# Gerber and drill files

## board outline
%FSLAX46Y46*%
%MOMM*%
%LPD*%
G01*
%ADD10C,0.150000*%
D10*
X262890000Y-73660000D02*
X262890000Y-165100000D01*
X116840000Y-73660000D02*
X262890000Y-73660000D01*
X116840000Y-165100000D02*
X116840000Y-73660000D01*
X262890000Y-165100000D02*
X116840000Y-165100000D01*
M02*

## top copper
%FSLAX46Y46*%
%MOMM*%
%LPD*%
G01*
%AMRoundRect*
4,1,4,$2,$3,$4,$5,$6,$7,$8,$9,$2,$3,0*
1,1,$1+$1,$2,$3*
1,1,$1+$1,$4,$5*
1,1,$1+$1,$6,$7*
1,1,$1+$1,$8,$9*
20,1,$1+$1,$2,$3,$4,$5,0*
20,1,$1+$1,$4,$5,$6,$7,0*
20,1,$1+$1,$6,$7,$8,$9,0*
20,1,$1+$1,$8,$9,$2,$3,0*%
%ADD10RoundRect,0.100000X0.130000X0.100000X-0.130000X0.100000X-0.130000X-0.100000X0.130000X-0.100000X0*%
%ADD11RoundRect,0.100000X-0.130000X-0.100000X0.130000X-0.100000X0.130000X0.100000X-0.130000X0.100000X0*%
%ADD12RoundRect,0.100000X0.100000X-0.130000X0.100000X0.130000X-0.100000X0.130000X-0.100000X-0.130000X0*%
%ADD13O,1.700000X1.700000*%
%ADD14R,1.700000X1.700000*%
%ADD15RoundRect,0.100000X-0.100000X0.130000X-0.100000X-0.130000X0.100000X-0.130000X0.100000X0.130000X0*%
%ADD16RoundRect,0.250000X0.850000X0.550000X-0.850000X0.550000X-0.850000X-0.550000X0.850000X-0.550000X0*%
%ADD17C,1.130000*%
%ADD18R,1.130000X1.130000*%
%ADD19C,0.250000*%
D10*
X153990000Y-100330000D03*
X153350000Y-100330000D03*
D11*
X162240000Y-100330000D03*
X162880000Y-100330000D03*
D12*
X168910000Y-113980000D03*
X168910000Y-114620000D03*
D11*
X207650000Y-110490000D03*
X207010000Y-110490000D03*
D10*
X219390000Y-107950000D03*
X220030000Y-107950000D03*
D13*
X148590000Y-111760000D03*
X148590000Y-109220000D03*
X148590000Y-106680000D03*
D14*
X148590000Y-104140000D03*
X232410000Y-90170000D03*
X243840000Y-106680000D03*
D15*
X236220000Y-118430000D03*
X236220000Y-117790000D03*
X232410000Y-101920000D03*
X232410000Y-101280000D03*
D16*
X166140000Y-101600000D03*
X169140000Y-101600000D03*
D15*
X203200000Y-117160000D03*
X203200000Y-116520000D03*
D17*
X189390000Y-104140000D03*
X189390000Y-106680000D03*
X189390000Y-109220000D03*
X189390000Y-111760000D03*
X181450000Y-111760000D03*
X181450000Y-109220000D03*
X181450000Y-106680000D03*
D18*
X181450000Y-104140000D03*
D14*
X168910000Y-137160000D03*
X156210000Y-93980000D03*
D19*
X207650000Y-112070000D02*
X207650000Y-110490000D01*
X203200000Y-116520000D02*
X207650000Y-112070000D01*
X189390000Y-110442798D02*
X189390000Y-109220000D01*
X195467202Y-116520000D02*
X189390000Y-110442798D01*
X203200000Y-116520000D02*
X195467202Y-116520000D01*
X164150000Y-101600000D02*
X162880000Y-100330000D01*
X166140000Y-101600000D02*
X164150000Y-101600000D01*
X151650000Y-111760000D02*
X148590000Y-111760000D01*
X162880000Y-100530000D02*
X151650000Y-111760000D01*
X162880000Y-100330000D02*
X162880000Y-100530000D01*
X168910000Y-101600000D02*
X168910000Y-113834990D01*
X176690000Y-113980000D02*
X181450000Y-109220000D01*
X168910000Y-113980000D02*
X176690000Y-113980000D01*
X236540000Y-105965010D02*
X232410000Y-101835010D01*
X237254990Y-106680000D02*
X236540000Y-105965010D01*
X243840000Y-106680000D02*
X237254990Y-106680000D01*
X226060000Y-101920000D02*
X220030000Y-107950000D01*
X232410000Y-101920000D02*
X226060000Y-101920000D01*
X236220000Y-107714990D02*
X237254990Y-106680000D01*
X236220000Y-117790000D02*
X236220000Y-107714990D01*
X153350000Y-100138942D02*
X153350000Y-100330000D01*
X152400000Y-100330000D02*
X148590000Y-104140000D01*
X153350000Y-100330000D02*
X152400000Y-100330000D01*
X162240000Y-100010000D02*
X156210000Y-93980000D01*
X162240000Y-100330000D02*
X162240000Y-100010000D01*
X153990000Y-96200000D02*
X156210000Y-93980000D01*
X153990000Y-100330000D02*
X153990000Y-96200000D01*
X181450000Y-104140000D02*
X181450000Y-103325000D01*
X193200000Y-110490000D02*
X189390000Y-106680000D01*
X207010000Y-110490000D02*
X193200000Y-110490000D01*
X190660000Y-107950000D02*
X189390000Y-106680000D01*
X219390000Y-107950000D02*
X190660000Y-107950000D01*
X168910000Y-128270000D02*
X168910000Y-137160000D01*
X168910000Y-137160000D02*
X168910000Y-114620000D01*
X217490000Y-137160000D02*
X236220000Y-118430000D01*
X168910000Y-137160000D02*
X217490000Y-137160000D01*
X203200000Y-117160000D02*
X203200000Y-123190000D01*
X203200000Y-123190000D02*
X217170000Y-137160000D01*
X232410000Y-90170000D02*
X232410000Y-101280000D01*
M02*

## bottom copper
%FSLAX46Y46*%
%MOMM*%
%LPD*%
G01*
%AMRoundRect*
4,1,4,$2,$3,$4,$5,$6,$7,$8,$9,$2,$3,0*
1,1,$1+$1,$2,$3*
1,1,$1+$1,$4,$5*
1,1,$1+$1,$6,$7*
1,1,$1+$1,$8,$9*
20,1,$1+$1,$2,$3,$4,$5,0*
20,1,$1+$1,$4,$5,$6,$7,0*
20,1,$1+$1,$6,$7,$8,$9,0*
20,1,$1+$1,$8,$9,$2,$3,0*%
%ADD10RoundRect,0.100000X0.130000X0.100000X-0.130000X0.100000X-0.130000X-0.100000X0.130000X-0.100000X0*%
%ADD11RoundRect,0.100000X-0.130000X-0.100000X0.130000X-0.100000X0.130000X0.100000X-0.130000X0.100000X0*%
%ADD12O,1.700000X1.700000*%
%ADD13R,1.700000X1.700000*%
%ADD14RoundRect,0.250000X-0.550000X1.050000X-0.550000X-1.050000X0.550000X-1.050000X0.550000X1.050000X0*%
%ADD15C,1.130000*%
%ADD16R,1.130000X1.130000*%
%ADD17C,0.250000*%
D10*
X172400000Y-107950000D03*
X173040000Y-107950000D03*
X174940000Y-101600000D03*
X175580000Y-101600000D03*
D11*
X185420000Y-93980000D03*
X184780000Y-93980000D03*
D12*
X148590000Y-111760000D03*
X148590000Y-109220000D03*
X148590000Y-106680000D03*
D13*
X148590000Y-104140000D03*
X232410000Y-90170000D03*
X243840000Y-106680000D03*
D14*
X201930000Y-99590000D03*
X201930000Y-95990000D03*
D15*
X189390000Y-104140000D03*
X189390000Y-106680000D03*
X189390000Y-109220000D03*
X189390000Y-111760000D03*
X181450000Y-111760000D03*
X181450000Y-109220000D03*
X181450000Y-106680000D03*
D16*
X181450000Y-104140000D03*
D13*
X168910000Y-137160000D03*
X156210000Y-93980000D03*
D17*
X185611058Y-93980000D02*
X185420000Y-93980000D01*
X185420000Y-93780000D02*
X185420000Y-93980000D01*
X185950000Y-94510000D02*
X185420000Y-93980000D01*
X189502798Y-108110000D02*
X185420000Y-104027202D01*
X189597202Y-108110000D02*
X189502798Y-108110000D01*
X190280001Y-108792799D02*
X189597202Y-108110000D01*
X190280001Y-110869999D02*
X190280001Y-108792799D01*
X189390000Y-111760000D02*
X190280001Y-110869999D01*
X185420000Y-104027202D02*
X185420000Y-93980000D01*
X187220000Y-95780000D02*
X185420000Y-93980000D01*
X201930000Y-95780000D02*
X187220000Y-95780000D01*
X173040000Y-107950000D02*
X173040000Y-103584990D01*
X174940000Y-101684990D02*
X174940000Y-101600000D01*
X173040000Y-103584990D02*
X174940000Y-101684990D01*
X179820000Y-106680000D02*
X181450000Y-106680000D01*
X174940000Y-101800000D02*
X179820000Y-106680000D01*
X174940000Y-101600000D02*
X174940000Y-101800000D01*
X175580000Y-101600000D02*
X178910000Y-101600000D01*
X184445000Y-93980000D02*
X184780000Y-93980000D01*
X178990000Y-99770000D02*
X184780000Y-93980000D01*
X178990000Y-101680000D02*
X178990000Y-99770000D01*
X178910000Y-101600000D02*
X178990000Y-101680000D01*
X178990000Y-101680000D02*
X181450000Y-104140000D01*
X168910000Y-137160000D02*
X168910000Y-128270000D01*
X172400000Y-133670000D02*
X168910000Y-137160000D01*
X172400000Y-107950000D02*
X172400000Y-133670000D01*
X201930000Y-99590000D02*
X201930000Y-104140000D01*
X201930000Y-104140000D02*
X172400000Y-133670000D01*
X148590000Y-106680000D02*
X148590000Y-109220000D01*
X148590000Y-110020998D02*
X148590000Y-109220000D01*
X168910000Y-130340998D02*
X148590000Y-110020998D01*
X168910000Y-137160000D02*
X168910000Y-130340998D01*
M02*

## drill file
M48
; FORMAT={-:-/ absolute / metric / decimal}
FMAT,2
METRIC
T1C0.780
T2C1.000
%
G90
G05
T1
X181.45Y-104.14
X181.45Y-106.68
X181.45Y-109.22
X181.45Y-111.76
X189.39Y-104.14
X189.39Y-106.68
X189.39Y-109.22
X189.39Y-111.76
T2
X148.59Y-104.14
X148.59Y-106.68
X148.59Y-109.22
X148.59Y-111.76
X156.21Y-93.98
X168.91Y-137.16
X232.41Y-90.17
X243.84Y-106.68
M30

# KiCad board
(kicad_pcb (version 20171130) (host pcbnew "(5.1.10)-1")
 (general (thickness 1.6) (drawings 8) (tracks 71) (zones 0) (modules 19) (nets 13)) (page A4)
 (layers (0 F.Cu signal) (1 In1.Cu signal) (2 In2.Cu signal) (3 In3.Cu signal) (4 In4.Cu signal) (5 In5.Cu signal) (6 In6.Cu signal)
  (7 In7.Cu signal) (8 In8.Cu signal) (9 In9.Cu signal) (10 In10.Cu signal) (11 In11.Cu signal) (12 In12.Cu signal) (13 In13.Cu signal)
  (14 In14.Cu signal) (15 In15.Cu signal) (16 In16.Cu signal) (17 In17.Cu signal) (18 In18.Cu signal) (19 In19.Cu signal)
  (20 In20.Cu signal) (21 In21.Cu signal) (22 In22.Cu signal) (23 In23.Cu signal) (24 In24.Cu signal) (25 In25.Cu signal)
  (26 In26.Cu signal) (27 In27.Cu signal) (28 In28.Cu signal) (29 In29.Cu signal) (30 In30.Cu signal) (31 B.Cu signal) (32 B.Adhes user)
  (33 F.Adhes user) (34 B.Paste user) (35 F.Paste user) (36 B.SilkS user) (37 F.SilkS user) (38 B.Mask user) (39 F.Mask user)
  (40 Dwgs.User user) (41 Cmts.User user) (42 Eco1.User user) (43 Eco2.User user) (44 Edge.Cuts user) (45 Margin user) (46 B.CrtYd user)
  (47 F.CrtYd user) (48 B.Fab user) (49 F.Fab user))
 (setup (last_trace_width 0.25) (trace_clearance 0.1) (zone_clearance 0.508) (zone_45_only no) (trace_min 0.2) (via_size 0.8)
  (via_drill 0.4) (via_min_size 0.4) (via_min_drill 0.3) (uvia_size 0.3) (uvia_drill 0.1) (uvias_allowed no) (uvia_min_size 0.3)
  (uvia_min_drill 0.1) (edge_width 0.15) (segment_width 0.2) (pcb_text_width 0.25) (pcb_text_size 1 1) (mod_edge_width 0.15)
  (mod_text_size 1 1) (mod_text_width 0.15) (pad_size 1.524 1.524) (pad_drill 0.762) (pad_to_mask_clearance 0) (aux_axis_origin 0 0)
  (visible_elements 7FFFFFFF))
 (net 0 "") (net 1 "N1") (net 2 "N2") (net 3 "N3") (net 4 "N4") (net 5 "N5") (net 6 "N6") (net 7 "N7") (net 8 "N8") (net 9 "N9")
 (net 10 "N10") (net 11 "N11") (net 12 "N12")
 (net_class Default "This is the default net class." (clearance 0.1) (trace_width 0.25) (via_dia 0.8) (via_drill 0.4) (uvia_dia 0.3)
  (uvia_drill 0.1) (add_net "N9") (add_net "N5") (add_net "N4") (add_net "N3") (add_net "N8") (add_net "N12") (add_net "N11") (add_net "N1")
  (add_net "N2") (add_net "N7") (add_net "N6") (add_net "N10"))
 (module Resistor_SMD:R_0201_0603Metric (layer F.Cu) (at 153.67 100.33 180)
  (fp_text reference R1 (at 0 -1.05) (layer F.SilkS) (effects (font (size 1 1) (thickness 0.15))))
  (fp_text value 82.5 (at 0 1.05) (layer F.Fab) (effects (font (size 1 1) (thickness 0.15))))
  (pad "" smd roundrect (at -0.345 0 180) (size 0.318 0.36) (layers F.Paste) (roundrect_rratio 0.25))
  (pad "" smd roundrect (at 0.345 0 180) (size 0.318 0.36) (layers F.Paste) (roundrect_rratio 0.25))
  (pad 1 smd roundrect (at -0.32 0 180) (size 0.46 0.4) (layers F.Cu F.Mask) (roundrect_rratio 0.25) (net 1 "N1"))
  (pad 2 smd roundrect (at 0.32 0 180) (size 0.46 0.4) (layers F.Cu F.Mask) (roundrect_rratio 0.25) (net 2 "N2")))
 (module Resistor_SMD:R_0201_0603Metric (layer F.Cu) (at 162.56 100.33)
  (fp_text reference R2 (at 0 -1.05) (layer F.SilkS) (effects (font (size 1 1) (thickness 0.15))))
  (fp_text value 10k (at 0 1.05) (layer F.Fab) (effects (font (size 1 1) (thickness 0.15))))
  (pad "" smd roundrect (at -0.345 0) (size 0.318 0.36) (layers F.Paste) (roundrect_rratio 0.25))
  (pad "" smd roundrect (at 0.345 0) (size 0.318 0.36) (layers F.Paste) (roundrect_rratio 0.25))
  (pad 1 smd roundrect (at -0.32 0) (size 0.46 0.4) (layers F.Cu F.Mask) (roundrect_rratio 0.25) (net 1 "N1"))
  (pad 2 smd roundrect (at 0.32 0) (size 0.46 0.4) (layers F.Cu F.Mask) (roundrect_rratio 0.25) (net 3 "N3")))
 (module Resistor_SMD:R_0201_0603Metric (layer F.Cu) (at 168.91 114.3 90)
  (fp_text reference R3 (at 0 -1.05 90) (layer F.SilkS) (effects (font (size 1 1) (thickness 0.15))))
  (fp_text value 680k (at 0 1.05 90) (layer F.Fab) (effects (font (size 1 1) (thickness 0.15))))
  (pad 2 smd roundrect (at 0.32 0 90) (size 0.46 0.4) (layers F.Cu F.Mask) (roundrect_rratio 0.25) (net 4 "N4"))
  (pad 1 smd roundrect (at -0.32 0 90) (size 0.46 0.4) (layers F.Cu F.Mask) (roundrect_rratio 0.25) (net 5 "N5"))
  (pad "" smd roundrect (at 0.345 0 90) (size 0.318 0.36) (layers F.Paste) (roundrect_rratio 0.25))
  (pad "" smd roundrect (at -0.345 0 90) (size 0.318 0.36) (layers F.Paste) (roundrect_rratio 0.25)))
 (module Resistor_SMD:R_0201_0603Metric (layer B.Cu) (at 172.72 107.95 180)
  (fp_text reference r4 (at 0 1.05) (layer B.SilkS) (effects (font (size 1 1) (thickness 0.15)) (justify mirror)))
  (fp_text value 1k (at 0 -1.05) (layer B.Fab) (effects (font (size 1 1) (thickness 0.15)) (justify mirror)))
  (pad 2 smd roundrect (at 0.32 0 180) (size 0.46 0.4) (layers B.Cu B.Mask) (roundrect_rratio 0.25) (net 5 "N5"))
  (pad 1 smd roundrect (at -0.32 0 180) (size 0.46 0.4) (layers B.Cu B.Mask) (roundrect_rratio 0.25) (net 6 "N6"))
  (pad "" smd roundrect (at 0.345 0 180) (size 0.318 0.36) (layers B.Paste) (roundrect_rratio 0.25))
  (pad "" smd roundrect (at -0.345 0 180) (size 0.318 0.36) (layers B.Paste) (roundrect_rratio 0.25)))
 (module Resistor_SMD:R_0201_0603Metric (layer B.Cu) (at 175.26 101.6 180)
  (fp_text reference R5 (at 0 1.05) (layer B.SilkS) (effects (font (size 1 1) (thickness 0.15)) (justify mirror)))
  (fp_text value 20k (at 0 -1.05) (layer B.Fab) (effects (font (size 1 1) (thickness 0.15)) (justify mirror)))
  (pad 2 smd roundrect (at 0.32 0 180) (size 0.46 0.4) (layers B.Cu B.Mask) (roundrect_rratio 0.25) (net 6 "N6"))
  (pad 1 smd roundrect (at -0.32 0 180) (size 0.46 0.4) (layers B.Cu B.Mask) (roundrect_rratio 0.25) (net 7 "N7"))
  (pad "" smd roundrect (at 0.345 0 180) (size 0.318 0.36) (layers B.Paste) (roundrect_rratio 0.25))
  (pad "" smd roundrect (at -0.345 0 180) (size 0.318 0.36) (layers B.Paste) (roundrect_rratio 0.25)))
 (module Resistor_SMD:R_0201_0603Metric (layer B.Cu) (at 185.1 93.98)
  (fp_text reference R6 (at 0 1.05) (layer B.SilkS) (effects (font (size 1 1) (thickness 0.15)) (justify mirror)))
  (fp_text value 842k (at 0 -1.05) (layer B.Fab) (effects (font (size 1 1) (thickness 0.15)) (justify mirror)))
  (pad 2 smd roundrect (at 0.32 0) (size 0.46 0.4) (layers B.Cu B.Mask) (roundrect_rratio 0.25) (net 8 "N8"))
  (pad 1 smd roundrect (at -0.32 0) (size 0.46 0.4) (layers B.Cu B.Mask) (roundrect_rratio 0.25) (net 7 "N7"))
  (pad "" smd roundrect (at 0.345 0) (size 0.318 0.36) (layers B.Paste) (roundrect_rratio 0.25))
  (pad "" smd roundrect (at -0.345 0) (size 0.318 0.36) (layers B.Paste) (roundrect_rratio 0.25)))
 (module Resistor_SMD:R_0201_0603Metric (layer F.Cu) (at 207.33 110.49)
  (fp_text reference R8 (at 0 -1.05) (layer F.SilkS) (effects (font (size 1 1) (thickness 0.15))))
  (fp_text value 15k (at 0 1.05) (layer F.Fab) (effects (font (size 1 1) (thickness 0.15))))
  (pad 2 smd roundrect (at 0.32 0) (size 0.46 0.4) (layers F.Cu F.Mask) (roundrect_rratio 0.25) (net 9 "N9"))
  (pad 1 smd roundrect (at -0.32 0) (size 0.46 0.4) (layers F.Cu F.Mask) (roundrect_rratio 0.25) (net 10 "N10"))
  (pad "" smd roundrect (at 0.345 0) (size 0.318 0.36) (layers F.Paste) (roundrect_rratio 0.25))
  (pad "" smd roundrect (at -0.345 0) (size 0.318 0.36) (layers F.Paste) (roundrect_rratio 0.25)))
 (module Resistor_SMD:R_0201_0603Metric (layer F.Cu) (at 219.71 107.95 180)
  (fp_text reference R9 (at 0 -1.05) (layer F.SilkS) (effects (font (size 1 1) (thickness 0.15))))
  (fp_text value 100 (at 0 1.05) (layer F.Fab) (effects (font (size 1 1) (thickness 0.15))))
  (pad 2 smd roundrect (at 0.32 0 180) (size 0.46 0.4) (layers F.Cu F.Mask) (roundrect_rratio 0.25) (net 10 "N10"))
  (pad 1 smd roundrect (at -0.32 0 180) (size 0.46 0.4) (layers F.Cu F.Mask) (roundrect_rratio 0.25) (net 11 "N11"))
  (pad "" smd roundrect (at 0.345 0 180) (size 0.318 0.36) (layers F.Paste) (roundrect_rratio 0.25))
  (pad "" smd roundrect (at -0.345 0 180) (size 0.318 0.36) (layers F.Paste) (roundrect_rratio 0.25)))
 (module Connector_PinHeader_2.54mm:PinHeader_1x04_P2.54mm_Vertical (layer F.Cu) (at 148.59 104.14)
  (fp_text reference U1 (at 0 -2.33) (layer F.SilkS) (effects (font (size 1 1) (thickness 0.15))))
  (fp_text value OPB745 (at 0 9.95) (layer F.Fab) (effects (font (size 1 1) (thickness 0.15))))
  (pad 4 thru_hole oval (at 0 7.62) (size 1.7 1.7) (drill 1) (layers *.Cu *.Mask) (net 3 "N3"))
  (pad 3 thru_hole oval (at 0 5.08) (size 1.7 1.7) (drill 1) (layers *.Cu *.Mask) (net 5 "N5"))
  (pad 2 thru_hole oval (at 0 2.54) (size 1.7 1.7) (drill 1) (layers *.Cu *.Mask) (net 5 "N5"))
  (pad 1 thru_hole rect (at 0 0) (size 1.7 1.7) (drill 1) (layers *.Cu *.Mask) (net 2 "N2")))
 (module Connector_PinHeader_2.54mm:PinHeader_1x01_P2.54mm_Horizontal (layer F.Cu) (at 232.41 90.17 90)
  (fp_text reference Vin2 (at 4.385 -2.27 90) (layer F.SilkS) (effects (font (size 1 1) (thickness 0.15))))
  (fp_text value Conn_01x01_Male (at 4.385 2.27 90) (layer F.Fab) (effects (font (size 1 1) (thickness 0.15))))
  (pad 1 thru_hole rect (at 0 0 90) (size 1.7 1.7) (drill 1) (layers *.Cu *.Mask) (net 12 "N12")))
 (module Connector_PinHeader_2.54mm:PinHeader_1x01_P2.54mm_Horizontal (layer F.Cu) (at 243.84 106.68)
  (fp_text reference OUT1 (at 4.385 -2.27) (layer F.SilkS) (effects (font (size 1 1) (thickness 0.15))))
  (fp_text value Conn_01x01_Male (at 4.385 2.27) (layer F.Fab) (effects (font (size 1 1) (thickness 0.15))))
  (pad 1 thru_hole rect (at 0 0) (size 1.7 1.7) (drill 1) (layers *.Cu *.Mask) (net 11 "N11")))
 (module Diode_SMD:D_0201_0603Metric (layer F.Cu) (at 236.22 118.11 270)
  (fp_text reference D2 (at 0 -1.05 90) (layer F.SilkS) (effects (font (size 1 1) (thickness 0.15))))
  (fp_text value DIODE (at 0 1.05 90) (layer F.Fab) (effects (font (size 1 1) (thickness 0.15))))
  (pad 2 smd roundrect (at 0.32 0 270) (size 0.46 0.4) (layers F.Cu F.Mask) (roundrect_rratio 0.25) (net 5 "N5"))
  (pad 1 smd roundrect (at -0.32 0 270) (size 0.46 0.4) (layers F.Cu F.Mask) (roundrect_rratio 0.25) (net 11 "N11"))
  (pad "" smd roundrect (at 0.345 0 270) (size 0.318 0.36) (layers F.Paste) (roundrect_rratio 0.25))
  (pad "" smd roundrect (at -0.345 0 270) (size 0.318 0.36) (layers F.Paste) (roundrect_rratio 0.25)))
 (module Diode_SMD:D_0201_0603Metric (layer F.Cu) (at 232.41 101.6 270)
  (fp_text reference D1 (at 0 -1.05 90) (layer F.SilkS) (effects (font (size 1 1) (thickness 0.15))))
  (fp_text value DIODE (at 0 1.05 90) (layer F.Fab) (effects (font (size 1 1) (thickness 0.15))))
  (pad 2 smd roundrect (at 0.32 0 270) (size 0.46 0.4) (layers F.Cu F.Mask) (roundrect_rratio 0.25) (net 11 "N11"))
  (pad 1 smd roundrect (at -0.32 0 270) (size 0.46 0.4) (layers F.Cu F.Mask) (roundrect_rratio 0.25) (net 12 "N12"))
  (pad "" smd roundrect (at 0.345 0 270) (size 0.318 0.36) (layers F.Paste) (roundrect_rratio 0.25))
  (pad "" smd roundrect (at -0.345 0 270) (size 0.318 0.36) (layers F.Paste) (roundrect_rratio 0.25)))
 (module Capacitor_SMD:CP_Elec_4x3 (layer B.Cu) (at 201.93 97.79 270)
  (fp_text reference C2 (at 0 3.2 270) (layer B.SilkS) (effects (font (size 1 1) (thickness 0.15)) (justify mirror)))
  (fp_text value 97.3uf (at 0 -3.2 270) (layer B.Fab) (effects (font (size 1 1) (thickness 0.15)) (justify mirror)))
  (pad 2 smd roundrect (at 1.8 0 270) (size 2.6 1.6) (layers B.Cu B.Paste B.Mask) (roundrect_rratio 0.15625) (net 5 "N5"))
  (pad 1 smd roundrect (at -1.8 0 270) (size 2.6 1.6) (layers B.Cu B.Paste B.Mask) (roundrect_rratio 0.15625) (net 8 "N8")))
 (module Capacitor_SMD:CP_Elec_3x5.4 (layer F.Cu) (at 167.64 101.6 180)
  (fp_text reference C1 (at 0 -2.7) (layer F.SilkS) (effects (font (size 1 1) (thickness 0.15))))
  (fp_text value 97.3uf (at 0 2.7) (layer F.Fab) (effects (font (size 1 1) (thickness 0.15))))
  (pad 2 smd roundrect (at 1.5 0 180) (size 2.2 1.6) (layers F.Cu F.Paste F.Mask) (roundrect_rratio 0.15625) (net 3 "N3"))
  (pad 1 smd roundrect (at -1.5 0 180) (size 2.2 1.6) (layers F.Cu F.Paste F.Mask) (roundrect_rratio 0.15625) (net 4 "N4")))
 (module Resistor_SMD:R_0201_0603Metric (layer F.Cu) (at 203.2 116.84 270)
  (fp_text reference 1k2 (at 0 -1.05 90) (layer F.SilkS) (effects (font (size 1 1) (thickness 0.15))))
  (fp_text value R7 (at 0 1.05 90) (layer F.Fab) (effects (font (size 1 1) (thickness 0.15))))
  (pad 2 smd roundrect (at 0.32 0 270) (size 0.46 0.4) (layers F.Cu F.Mask) (roundrect_rratio 0.25) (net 5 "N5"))
  (pad 1 smd roundrect (at -0.32 0 270) (size 0.46 0.4) (layers F.Cu F.Mask) (roundrect_rratio 0.25) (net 9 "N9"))
  (pad "" smd roundrect (at 0.345 0 270) (size 0.318 0.36) (layers F.Paste) (roundrect_rratio 0.25))
  (pad "" smd roundrect (at -0.345 0 270) (size 0.318 0.36) (layers F.Paste) (roundrect_rratio 0.25)))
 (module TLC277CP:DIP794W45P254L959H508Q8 (layer F.Cu) (at 185.42 107.95)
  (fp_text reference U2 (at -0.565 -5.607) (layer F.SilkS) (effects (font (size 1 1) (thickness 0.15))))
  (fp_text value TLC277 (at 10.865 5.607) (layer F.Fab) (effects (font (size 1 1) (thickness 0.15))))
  (pad 8 thru_hole circle (at 3.97 -3.81) (size 1.13 1.13) (drill 0.78) (layers *.Cu *.Mask))
  (pad 7 thru_hole circle (at 3.97 -1.27) (size 1.13 1.13) (drill 0.78) (layers *.Cu *.Mask) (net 10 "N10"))
  (pad 6 thru_hole circle (at 3.97 1.27) (size 1.13 1.13) (drill 0.78) (layers *.Cu *.Mask) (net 9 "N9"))
  (pad 5 thru_hole circle (at 3.97 3.81) (size 1.13 1.13) (drill 0.78) (layers *.Cu *.Mask) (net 8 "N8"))
  (pad 4 thru_hole circle (at -3.97 3.81) (size 1.13 1.13) (drill 0.78) (layers *.Cu *.Mask))
  (pad 3 thru_hole circle (at -3.97 1.27) (size 1.13 1.13) (drill 0.78) (layers *.Cu *.Mask) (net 4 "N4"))
  (pad 2 thru_hole circle (at -3.97 -1.27) (size 1.13 1.13) (drill 0.78) (layers *.Cu *.Mask) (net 6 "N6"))
  (pad 1 thru_hole rect (at -3.97 -3.81) (size 1.13 1.13) (drill 0.78) (layers *.Cu *.Mask) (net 7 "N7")))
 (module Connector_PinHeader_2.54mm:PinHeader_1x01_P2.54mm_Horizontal (layer F.Cu) (at 168.91 137.16 270)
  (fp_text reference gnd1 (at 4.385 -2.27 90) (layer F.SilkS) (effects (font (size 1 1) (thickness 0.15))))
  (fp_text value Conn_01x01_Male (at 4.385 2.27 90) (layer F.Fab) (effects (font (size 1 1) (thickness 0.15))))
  (pad 1 thru_hole rect (at 0 0 270) (size 1.7 1.7) (drill 1) (layers *.Cu *.Mask) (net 5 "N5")))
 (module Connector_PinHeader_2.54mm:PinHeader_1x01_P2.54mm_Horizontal (layer F.Cu) (at 156.21 93.98 90)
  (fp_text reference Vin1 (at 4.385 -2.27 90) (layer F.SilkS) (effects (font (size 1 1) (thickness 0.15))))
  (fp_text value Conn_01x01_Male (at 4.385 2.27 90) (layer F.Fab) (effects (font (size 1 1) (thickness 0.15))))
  (pad 1 thru_hole rect (at 0 0 90) (size 1.7 1.7) (drill 1) (layers *.Cu *.Mask) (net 1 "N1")))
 (gr_line (start 262.89 73.66) (end 262.89 165.1) (layer Edge.Cuts) (width 0.15))
 (gr_line (start 116.84 73.66) (end 262.89 73.66) (layer Edge.Cuts) (width 0.15))
 (gr_line (start 116.84 165.1) (end 116.84 73.66) (layer Edge.Cuts) (width 0.15))
 (gr_line (start 262.89 165.1) (end 116.84 165.1) (layer Edge.Cuts) (width 0.15))
 (segment (start 207.65 112.07) (end 207.65 110.49) (width 0.25) (layer F.Cu) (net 9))
 (segment (start 203.2 116.52) (end 207.65 112.07) (width 0.25) (layer F.Cu) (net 9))
 (segment (start 189.39 110.442798) (end 189.39 109.22) (width 0.25) (layer F.Cu) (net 9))
 (segment (start 195.467202 116.52) (end 189.39 110.442798) (width 0.25) (layer F.Cu) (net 9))
 (segment (start 203.2 116.52) (end 195.467202 116.52) (width 0.25) (layer F.Cu) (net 9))
 (segment (start 164.15 101.6) (end 162.88 100.33) (width 0.25) (layer F.Cu) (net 3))
 (segment (start 166.14 101.6) (end 164.15 101.6) (width 0.25) (layer F.Cu) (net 3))
 (segment (start 151.65 111.76) (end 148.59 111.76) (width 0.25) (layer F.Cu) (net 3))
 (segment (start 162.88 100.53) (end 151.65 111.76) (width 0.25) (layer F.Cu) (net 3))
 (segment (start 162.88 100.33) (end 162.88 100.53) (width 0.25) (layer F.Cu) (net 3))
 (segment (start 168.91 101.6) (end 168.91 113.83499) (width 0.25) (layer F.Cu) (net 4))
 (segment (start 176.69 113.98) (end 181.45 109.22) (width 0.25) (layer F.Cu) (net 4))
 (segment (start 168.91 113.98) (end 176.69 113.98) (width 0.25) (layer F.Cu) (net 4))
 (segment (start 185.611058 93.98) (end 185.42 93.98) (width 0.25) (layer B.Cu) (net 8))
 (segment (start 185.42 93.78) (end 185.42 93.98) (width 0.25) (layer B.Cu) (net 8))
 (segment (start 185.95 94.51) (end 185.42 93.98) (width 0.25) (layer B.Cu) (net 8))
 (segment (start 189.502798 108.11) (end 185.42 104.027202) (width 0.25) (layer B.Cu) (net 8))
 (segment (start 189.597202 108.11) (end 189.502798 108.11) (width 0.25) (layer B.Cu) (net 8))
 (segment (start 190.280001 108.792799) (end 189.597202 108.11) (width 0.25) (layer B.Cu) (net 8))
 (segment (start 190.280001 110.869999) (end 190.280001 108.792799) (width 0.25) (layer B.Cu) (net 8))
 (segment (start 189.39 111.76) (end 190.280001 110.869999) (width 0.25) (layer B.Cu) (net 8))
 (segment (start 185.42 104.027202) (end 185.42 93.98) (width 0.25) (layer B.Cu) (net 8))
 (segment (start 187.22 95.78) (end 185.42 93.98) (width 0.25) (layer B.Cu) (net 8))
 (segment (start 201.93 95.78) (end 187.22 95.78) (width 0.25) (layer B.Cu) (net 8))
 (segment (start 236.54 105.96501) (end 232.41 101.83501) (width 0.25) (layer F.Cu) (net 11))
 (segment (start 237.25499 106.68) (end 236.54 105.96501) (width 0.25) (layer F.Cu) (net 11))
 (segment (start 243.84 106.68) (end 237.25499 106.68) (width 0.25) (layer F.Cu) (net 11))
 (segment (start 226.06 101.92) (end 220.03 107.95) (width 0.25) (layer F.Cu) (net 11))
 (segment (start 232.41 101.92) (end 226.06 101.92) (width 0.25) (layer F.Cu) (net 11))
 (segment (start 236.22 107.71499) (end 237.25499 106.68) (width 0.25) (layer F.Cu) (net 11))
 (segment (start 236.22 117.79) (end 236.22 107.71499) (width 0.25) (layer F.Cu) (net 11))
 (segment (start 153.35 100.138942) (end 153.35 100.33) (width 0.25) (layer F.Cu) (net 2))
 (segment (start 152.4 100.33) (end 148.59 104.14) (width 0.25) (layer F.Cu) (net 2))
 (segment (start 153.35 100.33) (end 152.4 100.33) (width 0.25) (layer F.Cu) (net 2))
 (segment (start 162.24 100.01) (end 156.21 93.98) (width 0.25) (layer F.Cu) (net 1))
 (segment (start 162.24 100.33) (end 162.24 100.01) (width 0.25) (layer F.Cu) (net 1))
 (segment (start 153.99 96.2) (end 156.21 93.98) (width 0.25) (layer F.Cu) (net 1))
 (segment (start 153.99 100.33) (end 153.99 96.2) (width 0.25) (layer F.Cu) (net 1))
 (segment (start 173.04 107.95) (end 173.04 103.58499) (width 0.25) (layer B.Cu) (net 6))
 (segment (start 174.94 101.68499) (end 174.94 101.6) (width 0.25) (layer B.Cu) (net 6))
 (segment (start 173.04 103.58499) (end 174.94 101.68499) (width 0.25) (layer B.Cu) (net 6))
 (segment (start 179.82 106.68) (end 181.45 106.68) (width 0.25) (layer B.Cu) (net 6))
 (segment (start 174.94 101.8) (end 179.82 106.68) (width 0.25) (layer B.Cu) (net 6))
 (segment (start 174.94 101.6) (end 174.94 101.8) (width 0.25) (layer B.Cu) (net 6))
 (segment (start 175.58 101.6) (end 178.91 101.6) (width 0.25) (layer B.Cu) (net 7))
 (segment (start 184.445 93.98) (end 184.78 93.98) (width 0.25) (layer B.Cu) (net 7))
 (segment (start 181.45 104.14) (end 181.45 103.325) (width 0.25) (layer F.Cu) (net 7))
 (segment (start 178.99 99.77) (end 184.78 93.98) (width 0.25) (layer B.Cu) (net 7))
 (segment (start 178.99 101.68) (end 178.99 99.77) (width 0.25) (layer B.Cu) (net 7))
 (segment (start 178.91 101.6) (end 178.99 101.68) (width 0.25) (layer B.Cu) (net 7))
 (segment (start 178.99 101.68) (end 181.45 104.14) (width 0.25) (layer B.Cu) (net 7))
 (segment (start 193.2 110.49) (end 189.39 106.68) (width 0.25) (layer F.Cu) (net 10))
 (segment (start 207.01 110.49) (end 193.2 110.49) (width 0.25) (layer F.Cu) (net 10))
 (segment (start 190.66 107.95) (end 189.39 106.68) (width 0.25) (layer F.Cu) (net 10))
 (segment (start 219.39 107.95) (end 190.66 107.95) (width 0.25) (layer F.Cu) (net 10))
 (segment (start 168.91 128.27) (end 168.91 137.16) (width 0.25) (layer F.Cu) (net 5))
 (segment (start 168.91 137.16) (end 168.91 114.62) (width 0.25) (layer F.Cu) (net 5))
 (segment (start 168.91 137.16) (end 168.91 128.27) (width 0.25) (layer B.Cu) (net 5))
 (segment (start 172.4 133.67) (end 168.91 137.16) (width 0.25) (layer B.Cu) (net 5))
 (segment (start 172.4 107.95) (end 172.4 133.67) (width 0.25) (layer B.Cu) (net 5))
 (segment (start 217.49 137.16) (end 236.22 118.43) (width 0.25) (layer F.Cu) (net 5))
 (segment (start 168.91 137.16) (end 217.49 137.16) (width 0.25) (layer F.Cu) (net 5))
 (segment (start 203.2 117.16) (end 203.2 123.19) (width 0.25) (layer F.Cu) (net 5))
 (segment (start 203.2 123.19) (end 217.17 137.16) (width 0.25) (layer F.Cu) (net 5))
 (segment (start 201.93 99.59) (end 201.93 104.14) (width 0.25) (layer B.Cu) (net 5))
 (segment (start 201.93 104.14) (end 172.4 133.67) (width 0.25) (layer B.Cu) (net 5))
 (segment (start 148.59 106.68) (end 148.59 109.22) (width 0.25) (layer B.Cu) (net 5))
 (segment (start 148.59 110.020998) (end 148.59 109.22) (width 0.25) (layer B.Cu) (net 5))
 (segment (start 168.91 130.340998) (end 148.59 110.020998) (width 0.25) (layer B.Cu) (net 5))
 (segment (start 168.91 137.16) (end 168.91 130.340998) (width 0.25) (layer B.Cu) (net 5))
 (segment (start 232.41 90.17) (end 232.41 101.28) (width 0.25) (layer F.Cu) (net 12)))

